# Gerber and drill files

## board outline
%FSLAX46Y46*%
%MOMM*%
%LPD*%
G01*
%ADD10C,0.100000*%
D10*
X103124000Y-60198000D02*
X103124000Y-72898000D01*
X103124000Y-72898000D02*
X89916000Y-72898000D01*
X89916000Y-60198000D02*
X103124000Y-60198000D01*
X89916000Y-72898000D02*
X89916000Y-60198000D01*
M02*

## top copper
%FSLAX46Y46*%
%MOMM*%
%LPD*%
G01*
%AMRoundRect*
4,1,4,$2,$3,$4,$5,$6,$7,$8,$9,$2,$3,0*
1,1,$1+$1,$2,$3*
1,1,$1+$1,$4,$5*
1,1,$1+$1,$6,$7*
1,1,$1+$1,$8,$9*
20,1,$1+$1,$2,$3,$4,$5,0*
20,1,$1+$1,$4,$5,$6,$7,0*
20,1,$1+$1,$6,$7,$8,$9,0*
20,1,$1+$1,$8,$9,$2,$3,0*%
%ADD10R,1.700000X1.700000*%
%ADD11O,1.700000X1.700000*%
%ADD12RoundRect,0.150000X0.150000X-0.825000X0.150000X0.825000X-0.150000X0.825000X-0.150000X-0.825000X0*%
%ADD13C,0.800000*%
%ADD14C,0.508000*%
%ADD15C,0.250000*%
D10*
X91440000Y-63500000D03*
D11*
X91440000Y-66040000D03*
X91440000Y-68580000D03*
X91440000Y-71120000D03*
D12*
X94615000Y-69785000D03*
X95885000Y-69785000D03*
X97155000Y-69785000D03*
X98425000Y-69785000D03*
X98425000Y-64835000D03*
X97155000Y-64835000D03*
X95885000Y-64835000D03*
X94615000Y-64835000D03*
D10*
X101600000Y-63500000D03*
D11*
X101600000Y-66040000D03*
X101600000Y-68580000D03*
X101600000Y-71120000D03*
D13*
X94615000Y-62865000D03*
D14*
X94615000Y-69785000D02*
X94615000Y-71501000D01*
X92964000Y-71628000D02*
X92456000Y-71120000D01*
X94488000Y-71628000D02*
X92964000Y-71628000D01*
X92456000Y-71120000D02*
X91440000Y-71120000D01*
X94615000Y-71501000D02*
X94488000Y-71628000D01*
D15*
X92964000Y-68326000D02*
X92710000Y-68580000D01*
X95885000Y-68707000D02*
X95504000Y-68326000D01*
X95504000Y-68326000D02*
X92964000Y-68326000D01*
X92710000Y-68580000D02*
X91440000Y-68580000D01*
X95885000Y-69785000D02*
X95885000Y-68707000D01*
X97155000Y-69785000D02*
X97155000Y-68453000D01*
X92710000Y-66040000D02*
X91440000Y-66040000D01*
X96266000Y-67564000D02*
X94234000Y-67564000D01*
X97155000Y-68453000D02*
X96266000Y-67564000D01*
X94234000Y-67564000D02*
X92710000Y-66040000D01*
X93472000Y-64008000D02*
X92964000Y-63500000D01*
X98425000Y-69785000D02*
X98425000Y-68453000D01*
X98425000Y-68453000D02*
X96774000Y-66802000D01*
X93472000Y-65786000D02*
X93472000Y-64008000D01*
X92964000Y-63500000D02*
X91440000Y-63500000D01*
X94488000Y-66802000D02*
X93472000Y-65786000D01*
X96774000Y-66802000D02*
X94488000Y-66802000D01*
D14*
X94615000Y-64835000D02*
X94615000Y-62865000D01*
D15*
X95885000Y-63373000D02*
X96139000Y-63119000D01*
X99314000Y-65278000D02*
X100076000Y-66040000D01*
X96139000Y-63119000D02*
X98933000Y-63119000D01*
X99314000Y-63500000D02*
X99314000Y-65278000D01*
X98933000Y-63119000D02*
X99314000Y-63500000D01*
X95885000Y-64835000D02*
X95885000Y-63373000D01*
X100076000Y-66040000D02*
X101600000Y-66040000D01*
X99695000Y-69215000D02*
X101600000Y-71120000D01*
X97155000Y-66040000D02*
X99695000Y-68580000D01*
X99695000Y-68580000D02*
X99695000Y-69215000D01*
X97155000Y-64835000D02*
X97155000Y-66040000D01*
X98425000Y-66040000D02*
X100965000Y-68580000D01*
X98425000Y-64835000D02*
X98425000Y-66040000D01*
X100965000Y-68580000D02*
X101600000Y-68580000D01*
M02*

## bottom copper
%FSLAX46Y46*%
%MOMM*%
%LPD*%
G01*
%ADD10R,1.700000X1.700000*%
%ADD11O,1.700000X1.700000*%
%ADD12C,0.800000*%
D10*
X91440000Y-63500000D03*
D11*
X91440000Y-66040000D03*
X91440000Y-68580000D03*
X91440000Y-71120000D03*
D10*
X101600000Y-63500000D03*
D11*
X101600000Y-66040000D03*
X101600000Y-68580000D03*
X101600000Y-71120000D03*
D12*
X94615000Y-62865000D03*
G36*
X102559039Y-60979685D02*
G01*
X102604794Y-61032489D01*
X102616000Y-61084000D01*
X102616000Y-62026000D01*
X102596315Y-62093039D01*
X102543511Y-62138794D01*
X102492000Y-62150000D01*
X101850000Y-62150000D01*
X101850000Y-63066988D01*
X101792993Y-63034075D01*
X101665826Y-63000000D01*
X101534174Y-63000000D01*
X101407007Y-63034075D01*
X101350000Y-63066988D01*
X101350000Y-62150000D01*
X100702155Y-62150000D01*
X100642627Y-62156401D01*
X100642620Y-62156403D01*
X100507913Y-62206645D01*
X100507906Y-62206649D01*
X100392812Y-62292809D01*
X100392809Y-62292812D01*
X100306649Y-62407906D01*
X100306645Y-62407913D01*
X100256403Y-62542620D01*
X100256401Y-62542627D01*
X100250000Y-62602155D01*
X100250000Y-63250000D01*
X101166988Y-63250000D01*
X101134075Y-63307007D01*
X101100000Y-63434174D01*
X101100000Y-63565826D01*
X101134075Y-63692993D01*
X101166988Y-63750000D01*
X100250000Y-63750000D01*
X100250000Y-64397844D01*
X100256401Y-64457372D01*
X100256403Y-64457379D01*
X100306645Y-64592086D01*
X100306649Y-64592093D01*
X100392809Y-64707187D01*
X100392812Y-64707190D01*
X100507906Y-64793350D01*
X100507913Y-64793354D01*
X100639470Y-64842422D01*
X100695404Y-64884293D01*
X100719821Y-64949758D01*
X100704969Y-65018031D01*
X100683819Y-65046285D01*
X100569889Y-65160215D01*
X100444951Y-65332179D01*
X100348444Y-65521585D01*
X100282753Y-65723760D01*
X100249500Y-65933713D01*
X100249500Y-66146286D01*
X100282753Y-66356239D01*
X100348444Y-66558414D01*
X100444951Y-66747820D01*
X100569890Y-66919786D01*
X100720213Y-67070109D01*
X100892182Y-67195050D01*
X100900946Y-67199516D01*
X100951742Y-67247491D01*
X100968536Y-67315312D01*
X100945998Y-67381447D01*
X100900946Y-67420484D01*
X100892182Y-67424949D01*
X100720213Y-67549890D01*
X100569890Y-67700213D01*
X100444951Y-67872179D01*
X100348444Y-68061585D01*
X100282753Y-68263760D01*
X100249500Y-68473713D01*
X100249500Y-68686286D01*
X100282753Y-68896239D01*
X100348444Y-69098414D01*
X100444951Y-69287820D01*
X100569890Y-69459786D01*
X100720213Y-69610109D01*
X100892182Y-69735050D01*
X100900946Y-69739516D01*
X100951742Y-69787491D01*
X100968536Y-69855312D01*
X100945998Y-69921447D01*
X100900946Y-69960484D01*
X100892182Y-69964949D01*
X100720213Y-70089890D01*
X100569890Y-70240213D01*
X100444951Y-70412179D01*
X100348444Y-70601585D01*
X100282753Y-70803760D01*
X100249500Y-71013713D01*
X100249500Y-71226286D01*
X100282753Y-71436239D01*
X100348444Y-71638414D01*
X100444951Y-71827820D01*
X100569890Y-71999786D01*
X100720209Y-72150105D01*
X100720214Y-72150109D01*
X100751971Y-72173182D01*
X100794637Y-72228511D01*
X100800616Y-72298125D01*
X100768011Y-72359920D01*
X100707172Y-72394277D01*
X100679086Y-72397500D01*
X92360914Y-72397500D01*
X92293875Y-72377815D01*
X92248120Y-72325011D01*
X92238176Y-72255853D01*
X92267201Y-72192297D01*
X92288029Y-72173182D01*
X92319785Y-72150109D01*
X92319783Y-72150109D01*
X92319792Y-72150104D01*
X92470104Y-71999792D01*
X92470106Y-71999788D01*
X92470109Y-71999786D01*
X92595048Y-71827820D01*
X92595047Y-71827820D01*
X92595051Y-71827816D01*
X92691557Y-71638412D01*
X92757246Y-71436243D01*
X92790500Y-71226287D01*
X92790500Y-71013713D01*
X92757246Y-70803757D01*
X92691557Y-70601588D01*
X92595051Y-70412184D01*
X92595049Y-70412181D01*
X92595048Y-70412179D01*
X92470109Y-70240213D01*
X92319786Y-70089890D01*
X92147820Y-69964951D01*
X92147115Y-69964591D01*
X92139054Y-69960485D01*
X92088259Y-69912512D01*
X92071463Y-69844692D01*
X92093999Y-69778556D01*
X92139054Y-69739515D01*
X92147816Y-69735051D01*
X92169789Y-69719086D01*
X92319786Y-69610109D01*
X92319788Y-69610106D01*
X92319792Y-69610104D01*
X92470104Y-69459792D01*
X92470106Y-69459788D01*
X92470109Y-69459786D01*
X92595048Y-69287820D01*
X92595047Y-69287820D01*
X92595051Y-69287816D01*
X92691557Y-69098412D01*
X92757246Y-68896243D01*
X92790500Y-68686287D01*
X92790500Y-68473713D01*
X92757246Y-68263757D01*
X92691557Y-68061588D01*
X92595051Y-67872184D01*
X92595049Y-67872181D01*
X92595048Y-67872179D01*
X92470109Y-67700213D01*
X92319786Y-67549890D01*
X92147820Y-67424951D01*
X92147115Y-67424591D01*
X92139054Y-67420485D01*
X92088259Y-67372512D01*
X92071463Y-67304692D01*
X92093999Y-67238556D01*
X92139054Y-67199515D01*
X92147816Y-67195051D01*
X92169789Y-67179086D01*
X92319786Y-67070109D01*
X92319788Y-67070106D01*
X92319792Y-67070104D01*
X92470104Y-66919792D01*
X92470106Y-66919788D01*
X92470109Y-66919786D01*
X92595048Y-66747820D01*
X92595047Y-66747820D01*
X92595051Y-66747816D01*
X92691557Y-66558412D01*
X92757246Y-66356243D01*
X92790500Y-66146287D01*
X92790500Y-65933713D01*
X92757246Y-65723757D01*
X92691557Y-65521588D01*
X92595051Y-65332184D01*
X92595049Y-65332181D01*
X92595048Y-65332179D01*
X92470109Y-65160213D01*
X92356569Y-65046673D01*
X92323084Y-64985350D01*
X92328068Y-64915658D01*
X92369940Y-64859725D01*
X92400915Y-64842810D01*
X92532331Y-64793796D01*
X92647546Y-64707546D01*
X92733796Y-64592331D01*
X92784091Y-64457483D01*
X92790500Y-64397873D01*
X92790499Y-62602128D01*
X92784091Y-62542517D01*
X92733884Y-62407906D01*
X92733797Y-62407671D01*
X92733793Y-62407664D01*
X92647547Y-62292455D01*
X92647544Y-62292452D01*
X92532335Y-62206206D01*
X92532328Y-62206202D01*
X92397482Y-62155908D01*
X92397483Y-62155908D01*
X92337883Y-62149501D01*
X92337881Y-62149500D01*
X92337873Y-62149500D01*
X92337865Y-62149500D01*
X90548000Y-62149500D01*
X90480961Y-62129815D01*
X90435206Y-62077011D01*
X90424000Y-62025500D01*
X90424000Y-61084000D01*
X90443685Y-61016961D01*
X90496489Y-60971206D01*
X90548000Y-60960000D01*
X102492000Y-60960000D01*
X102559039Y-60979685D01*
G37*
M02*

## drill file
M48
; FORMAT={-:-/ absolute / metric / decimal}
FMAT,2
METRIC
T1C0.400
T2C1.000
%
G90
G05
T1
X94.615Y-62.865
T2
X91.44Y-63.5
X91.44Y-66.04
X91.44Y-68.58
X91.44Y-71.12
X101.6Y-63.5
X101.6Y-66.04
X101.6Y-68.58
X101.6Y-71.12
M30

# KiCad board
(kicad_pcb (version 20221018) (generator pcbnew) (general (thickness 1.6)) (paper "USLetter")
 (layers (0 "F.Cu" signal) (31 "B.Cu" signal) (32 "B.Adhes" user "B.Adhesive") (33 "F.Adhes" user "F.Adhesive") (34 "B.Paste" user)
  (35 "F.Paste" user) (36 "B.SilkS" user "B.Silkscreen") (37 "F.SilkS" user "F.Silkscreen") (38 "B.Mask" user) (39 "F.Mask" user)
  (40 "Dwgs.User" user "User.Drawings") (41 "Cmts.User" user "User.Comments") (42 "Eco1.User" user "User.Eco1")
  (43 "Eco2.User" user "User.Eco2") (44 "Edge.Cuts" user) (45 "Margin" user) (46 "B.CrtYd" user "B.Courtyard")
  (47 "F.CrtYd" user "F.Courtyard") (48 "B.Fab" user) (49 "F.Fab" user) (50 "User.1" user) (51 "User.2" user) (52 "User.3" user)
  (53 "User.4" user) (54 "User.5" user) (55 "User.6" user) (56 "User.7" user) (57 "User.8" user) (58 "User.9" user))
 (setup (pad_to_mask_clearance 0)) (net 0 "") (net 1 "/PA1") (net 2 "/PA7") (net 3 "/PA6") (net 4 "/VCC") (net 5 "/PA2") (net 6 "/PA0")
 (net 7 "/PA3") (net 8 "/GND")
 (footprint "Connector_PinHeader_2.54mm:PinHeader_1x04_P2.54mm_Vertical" (layer "F.Cu") (at 91.44 63.5)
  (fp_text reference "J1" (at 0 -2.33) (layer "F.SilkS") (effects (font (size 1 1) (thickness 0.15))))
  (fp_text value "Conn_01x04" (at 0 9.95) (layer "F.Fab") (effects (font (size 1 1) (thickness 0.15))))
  (pad "1" thru_hole rect (at 0 0) (size 1.7 1.7) (drill 1) (layers "*.Cu" "*.Mask") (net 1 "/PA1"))
  (pad "2" thru_hole oval (at 0 2.54) (size 1.7 1.7) (drill 1) (layers "*.Cu" "*.Mask") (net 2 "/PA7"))
  (pad "3" thru_hole oval (at 0 5.08) (size 1.7 1.7) (drill 1) (layers "*.Cu" "*.Mask") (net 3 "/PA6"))
  (pad "4" thru_hole oval (at 0 7.62) (size 1.7 1.7) (drill 1) (layers "*.Cu" "*.Mask") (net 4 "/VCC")))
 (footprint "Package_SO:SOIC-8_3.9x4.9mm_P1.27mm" (layer "F.Cu") (at 96.52 67.31 90)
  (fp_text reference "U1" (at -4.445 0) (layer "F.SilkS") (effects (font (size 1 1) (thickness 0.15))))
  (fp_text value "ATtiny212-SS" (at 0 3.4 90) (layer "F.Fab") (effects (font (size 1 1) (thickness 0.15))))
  (pad "1" smd roundrect (at -2.475 -1.905 90) (size 1.95 0.6) (layers "F.Cu" "F.Paste" "F.Mask") (roundrect_rratio 0.25) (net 4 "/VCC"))
  (pad "2" smd roundrect (at -2.475 -0.635 90) (size 1.95 0.6) (layers "F.Cu" "F.Paste" "F.Mask") (roundrect_rratio 0.25) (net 3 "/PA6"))
  (pad "3" smd roundrect (at -2.475 0.635 90) (size 1.95 0.6) (layers "F.Cu" "F.Paste" "F.Mask") (roundrect_rratio 0.25) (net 2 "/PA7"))
  (pad "4" smd roundrect (at -2.475 1.905 90) (size 1.95 0.6) (layers "F.Cu" "F.Paste" "F.Mask") (roundrect_rratio 0.25) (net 1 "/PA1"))
  (pad "5" smd roundrect (at 2.475 1.905 90) (size 1.95 0.6) (layers "F.Cu" "F.Paste" "F.Mask") (roundrect_rratio 0.25) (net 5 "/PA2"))
  (pad "6" smd roundrect (at 2.475 0.635 90) (size 1.95 0.6) (layers "F.Cu" "F.Paste" "F.Mask") (roundrect_rratio 0.25) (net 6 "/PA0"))
  (pad "7" smd roundrect (at 2.475 -0.635 90) (size 1.95 0.6) (layers "F.Cu" "F.Paste" "F.Mask") (roundrect_rratio 0.25) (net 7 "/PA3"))
  (pad "8" smd roundrect (at 2.475 -1.905 90) (size 1.95 0.6) (layers "F.Cu" "F.Paste" "F.Mask") (roundrect_rratio 0.25) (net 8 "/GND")))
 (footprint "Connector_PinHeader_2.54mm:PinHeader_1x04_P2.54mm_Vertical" (layer "F.Cu") (at 101.6 63.5)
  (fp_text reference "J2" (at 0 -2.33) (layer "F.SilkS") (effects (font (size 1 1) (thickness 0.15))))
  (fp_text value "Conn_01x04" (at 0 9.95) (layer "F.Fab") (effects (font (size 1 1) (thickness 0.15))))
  (pad "1" thru_hole rect (at 0 0) (size 1.7 1.7) (drill 1) (layers "*.Cu" "*.Mask") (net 8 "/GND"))
  (pad "2" thru_hole oval (at 0 2.54) (size 1.7 1.7) (drill 1) (layers "*.Cu" "*.Mask") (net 7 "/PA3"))
  (pad "3" thru_hole oval (at 0 5.08) (size 1.7 1.7) (drill 1) (layers "*.Cu" "*.Mask") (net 5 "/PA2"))
  (pad "4" thru_hole oval (at 0 7.62) (size 1.7 1.7) (drill 1) (layers "*.Cu" "*.Mask") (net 6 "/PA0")))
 (gr_line (start 103.124 60.198) (end 103.124 72.898) (stroke (width 0.1) (type default)) (layer "Edge.Cuts"))
 (gr_line (start 103.124 72.898) (end 89.916 72.898) (stroke (width 0.1) (type default)) (layer "Edge.Cuts"))
 (gr_line (start 89.916 60.198) (end 103.124 60.198) (stroke (width 0.1) (type default)) (layer "Edge.Cuts"))
 (gr_line (start 89.916 72.898) (end 89.916 60.198) (stroke (width 0.1) (type default)) (layer "Edge.Cuts"))
 (segment (start 94.615 69.785) (end 94.615 71.501) (width 0.508) (layer "F.Cu") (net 4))
 (segment (start 92.964 71.628) (end 92.456 71.12) (width 0.508) (layer "F.Cu") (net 4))
 (segment (start 94.488 71.628) (end 92.964 71.628) (width 0.508) (layer "F.Cu") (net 4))
 (segment (start 92.456 71.12) (end 91.44 71.12) (width 0.508) (layer "F.Cu") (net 4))
 (segment (start 94.615 71.501) (end 94.488 71.628) (width 0.508) (layer "F.Cu") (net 4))
 (segment (start 92.964 68.326) (end 92.71 68.58) (width 0.25) (layer "F.Cu") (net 3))
 (segment (start 95.885 68.707) (end 95.504 68.326) (width 0.25) (layer "F.Cu") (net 3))
 (segment (start 95.504 68.326) (end 92.964 68.326) (width 0.25) (layer "F.Cu") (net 3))
 (segment (start 92.71 68.58) (end 91.44 68.58) (width 0.25) (layer "F.Cu") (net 3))
 (segment (start 95.885 69.785) (end 95.885 68.707) (width 0.25) (layer "F.Cu") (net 3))
 (segment (start 97.155 69.785) (end 97.155 68.453) (width 0.25) (layer "F.Cu") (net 2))
 (segment (start 92.71 66.04) (end 91.44 66.04) (width 0.25) (layer "F.Cu") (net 2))
 (segment (start 96.266 67.564) (end 94.234 67.564) (width 0.25) (layer "F.Cu") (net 2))
 (segment (start 97.155 68.453) (end 96.266 67.564) (width 0.25) (layer "F.Cu") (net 2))
 (segment (start 94.234 67.564) (end 92.71 66.04) (width 0.25) (layer "F.Cu") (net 2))
 (segment (start 93.472 64.008) (end 92.964 63.5) (width 0.25) (layer "F.Cu") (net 1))
 (segment (start 98.425 69.785) (end 98.425 68.453) (width 0.25) (layer "F.Cu") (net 1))
 (segment (start 98.425 68.453) (end 96.774 66.802) (width 0.25) (layer "F.Cu") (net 1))
 (segment (start 93.472 65.786) (end 93.472 64.008) (width 0.25) (layer "F.Cu") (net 1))
 (segment (start 92.964 63.5) (end 91.44 63.5) (width 0.25) (layer "F.Cu") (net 1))
 (segment (start 94.488 66.802) (end 93.472 65.786) (width 0.25) (layer "F.Cu") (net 1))
 (segment (start 96.774 66.802) (end 94.488 66.802) (width 0.25) (layer "F.Cu") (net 1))
 (segment (start 94.615 64.835) (end 94.615 62.865) (width 0.508) (layer "F.Cu") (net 8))
 (via (at 94.615 62.865) (size 0.8) (drill 0.4) (layers "F.Cu" "B.Cu") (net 8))
 (segment (start 95.885 63.373) (end 96.139 63.119) (width 0.25) (layer "F.Cu") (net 7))
 (segment (start 99.314 65.278) (end 100.076 66.04) (width 0.25) (layer "F.Cu") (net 7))
 (segment (start 96.139 63.119) (end 98.933 63.119) (width 0.25) (layer "F.Cu") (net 7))
 (segment (start 99.314 63.5) (end 99.314 65.278) (width 0.25) (layer "F.Cu") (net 7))
 (segment (start 98.933 63.119) (end 99.314 63.5) (width 0.25) (layer "F.Cu") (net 7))
 (segment (start 95.885 64.835) (end 95.885 63.373) (width 0.25) (layer "F.Cu") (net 7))
 (segment (start 100.076 66.04) (end 101.6 66.04) (width 0.25) (layer "F.Cu") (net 7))
 (segment (start 99.695 69.215) (end 101.6 71.12) (width 0.25) (layer "F.Cu") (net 6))
 (segment (start 97.155 66.04) (end 99.695 68.58) (width 0.25) (layer "F.Cu") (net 6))
 (segment (start 99.695 68.58) (end 99.695 69.215) (width 0.25) (layer "F.Cu") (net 6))
 (segment (start 97.155 64.835) (end 97.155 66.04) (width 0.25) (layer "F.Cu") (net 6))
 (segment (start 98.425 66.04) (end 100.965 68.58) (width 0.25) (layer "F.Cu") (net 5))
 (segment (start 98.425 64.835) (end 98.425 66.04) (width 0.25) (layer "F.Cu") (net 5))
 (segment (start 100.965 68.58) (end 101.6 68.58) (width 0.25) (layer "F.Cu") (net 5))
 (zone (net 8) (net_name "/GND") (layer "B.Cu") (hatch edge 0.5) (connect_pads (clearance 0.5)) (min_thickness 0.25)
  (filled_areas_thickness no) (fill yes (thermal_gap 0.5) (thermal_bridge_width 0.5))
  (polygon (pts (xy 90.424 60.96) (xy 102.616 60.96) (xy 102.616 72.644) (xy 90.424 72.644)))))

